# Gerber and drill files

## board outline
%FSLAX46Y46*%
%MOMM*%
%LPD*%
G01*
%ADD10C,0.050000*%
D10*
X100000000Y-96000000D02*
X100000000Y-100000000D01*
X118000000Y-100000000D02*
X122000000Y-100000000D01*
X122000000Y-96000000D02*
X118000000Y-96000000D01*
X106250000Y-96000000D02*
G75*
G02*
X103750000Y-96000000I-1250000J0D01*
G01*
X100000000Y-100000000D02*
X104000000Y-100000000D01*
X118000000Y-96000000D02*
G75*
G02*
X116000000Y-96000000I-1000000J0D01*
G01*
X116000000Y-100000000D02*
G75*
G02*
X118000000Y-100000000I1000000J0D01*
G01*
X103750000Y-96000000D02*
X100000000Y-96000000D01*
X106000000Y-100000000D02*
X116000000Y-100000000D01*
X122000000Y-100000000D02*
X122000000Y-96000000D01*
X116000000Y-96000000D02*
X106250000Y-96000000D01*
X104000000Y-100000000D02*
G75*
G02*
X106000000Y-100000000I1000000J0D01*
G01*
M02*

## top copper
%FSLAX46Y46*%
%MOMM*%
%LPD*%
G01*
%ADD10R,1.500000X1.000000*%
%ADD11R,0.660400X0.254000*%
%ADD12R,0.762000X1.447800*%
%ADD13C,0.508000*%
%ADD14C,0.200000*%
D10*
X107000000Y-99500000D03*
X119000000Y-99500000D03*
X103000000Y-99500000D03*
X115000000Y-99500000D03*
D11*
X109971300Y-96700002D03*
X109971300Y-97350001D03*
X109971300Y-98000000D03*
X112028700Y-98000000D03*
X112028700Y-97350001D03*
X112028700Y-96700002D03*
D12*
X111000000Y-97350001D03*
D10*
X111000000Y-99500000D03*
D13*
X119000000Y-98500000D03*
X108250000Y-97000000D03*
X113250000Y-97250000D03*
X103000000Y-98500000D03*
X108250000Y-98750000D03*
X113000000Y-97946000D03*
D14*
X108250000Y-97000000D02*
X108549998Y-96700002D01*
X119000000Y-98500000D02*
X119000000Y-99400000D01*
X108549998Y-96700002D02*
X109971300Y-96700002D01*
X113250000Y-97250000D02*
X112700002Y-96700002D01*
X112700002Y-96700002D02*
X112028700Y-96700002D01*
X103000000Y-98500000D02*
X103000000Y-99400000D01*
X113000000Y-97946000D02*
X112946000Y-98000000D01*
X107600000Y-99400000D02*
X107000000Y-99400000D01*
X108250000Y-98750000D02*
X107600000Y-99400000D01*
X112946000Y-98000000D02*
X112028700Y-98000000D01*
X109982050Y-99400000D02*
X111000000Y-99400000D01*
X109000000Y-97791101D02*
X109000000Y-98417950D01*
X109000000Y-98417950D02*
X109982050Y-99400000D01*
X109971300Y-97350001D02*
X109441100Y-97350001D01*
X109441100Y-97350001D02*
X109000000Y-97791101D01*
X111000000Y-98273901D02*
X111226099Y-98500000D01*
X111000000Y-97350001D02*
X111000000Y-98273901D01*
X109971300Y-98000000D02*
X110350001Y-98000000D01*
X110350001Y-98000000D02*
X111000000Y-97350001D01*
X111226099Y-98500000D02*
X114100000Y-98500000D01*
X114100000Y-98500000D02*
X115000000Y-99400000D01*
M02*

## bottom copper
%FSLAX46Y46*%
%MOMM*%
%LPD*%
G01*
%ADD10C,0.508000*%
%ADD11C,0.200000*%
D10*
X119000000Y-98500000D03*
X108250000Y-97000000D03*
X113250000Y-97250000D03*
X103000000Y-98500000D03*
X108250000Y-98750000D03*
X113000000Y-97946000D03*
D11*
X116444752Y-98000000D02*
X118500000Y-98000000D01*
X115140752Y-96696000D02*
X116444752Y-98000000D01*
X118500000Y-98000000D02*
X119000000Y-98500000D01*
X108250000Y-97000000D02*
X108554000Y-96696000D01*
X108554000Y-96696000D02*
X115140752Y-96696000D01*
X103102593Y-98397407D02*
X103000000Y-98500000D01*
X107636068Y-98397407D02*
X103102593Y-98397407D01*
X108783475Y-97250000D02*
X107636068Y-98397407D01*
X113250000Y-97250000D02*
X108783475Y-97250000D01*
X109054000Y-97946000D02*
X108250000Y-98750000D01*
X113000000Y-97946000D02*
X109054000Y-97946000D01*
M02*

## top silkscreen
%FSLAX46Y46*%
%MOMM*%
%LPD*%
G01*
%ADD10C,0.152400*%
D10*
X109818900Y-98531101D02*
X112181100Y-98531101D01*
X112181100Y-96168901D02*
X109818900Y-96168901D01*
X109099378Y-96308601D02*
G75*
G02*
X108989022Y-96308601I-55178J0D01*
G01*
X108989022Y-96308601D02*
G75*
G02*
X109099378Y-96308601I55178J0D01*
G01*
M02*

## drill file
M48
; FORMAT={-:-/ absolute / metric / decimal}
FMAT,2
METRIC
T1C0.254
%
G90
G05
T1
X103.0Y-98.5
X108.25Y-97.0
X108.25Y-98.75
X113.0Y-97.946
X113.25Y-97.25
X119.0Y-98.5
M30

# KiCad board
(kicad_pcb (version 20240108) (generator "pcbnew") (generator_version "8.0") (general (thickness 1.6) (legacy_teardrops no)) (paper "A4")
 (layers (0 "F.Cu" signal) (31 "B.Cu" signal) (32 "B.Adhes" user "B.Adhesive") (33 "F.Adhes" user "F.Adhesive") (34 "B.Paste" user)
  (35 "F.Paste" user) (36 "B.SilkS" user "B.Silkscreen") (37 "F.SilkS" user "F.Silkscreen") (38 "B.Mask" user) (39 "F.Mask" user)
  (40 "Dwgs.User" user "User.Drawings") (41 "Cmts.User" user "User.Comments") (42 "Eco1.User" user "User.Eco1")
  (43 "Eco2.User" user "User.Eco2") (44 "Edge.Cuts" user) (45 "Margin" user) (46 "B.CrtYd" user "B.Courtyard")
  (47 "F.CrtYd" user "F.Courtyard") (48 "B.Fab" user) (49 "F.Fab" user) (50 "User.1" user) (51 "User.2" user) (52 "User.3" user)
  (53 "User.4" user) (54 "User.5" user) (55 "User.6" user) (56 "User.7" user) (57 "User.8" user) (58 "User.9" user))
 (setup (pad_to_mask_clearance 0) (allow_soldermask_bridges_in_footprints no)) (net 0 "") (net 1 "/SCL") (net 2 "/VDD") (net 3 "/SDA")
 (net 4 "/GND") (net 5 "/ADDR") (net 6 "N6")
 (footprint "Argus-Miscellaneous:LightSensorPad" (layer "F.Cu") (at 107 100.5)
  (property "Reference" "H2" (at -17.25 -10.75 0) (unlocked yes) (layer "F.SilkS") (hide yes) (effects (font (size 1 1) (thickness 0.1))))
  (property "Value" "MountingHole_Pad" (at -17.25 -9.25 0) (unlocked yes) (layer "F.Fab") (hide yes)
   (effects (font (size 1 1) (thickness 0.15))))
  (pad "1" smd rect (at 0 -1) (size 1.5 1) (layers "F.Cu" "F.Paste" "F.Mask") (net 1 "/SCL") (thermal_bridge_angle 45)))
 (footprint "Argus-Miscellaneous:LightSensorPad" (layer "F.Cu") (at 119 100.5)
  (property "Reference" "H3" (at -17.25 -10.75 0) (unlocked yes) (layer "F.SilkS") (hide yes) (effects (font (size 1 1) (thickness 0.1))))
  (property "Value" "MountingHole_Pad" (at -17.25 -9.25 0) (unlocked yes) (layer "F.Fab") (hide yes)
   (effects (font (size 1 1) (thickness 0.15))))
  (pad "1" smd rect (at 0 -1) (size 1.5 1) (layers "F.Cu" "F.Paste" "F.Mask") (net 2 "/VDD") (thermal_bridge_angle 45)))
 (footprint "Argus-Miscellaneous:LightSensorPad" (layer "F.Cu") (at 103 100.5)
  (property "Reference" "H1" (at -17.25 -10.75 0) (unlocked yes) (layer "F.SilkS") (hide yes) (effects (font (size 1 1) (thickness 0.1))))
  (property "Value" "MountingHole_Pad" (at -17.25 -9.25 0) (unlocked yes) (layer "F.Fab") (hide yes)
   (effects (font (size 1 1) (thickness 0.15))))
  (pad "1" smd rect (at 0 -1) (size 1.5 1) (layers "F.Cu" "F.Paste" "F.Mask") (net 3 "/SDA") (thermal_bridge_angle 45)))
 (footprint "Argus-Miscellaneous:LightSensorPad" (layer "F.Cu") (at 115 100.5)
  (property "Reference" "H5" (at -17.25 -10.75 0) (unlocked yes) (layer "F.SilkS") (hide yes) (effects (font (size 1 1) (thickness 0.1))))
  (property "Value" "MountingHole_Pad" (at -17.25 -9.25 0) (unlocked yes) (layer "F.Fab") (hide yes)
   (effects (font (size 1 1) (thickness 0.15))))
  (pad "1" smd rect (at 0 -1) (size 1.5 1) (layers "F.Cu" "F.Paste" "F.Mask") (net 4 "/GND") (thermal_bridge_angle 45)))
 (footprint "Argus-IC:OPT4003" (layer "F.Cu") (at 111 97.350001)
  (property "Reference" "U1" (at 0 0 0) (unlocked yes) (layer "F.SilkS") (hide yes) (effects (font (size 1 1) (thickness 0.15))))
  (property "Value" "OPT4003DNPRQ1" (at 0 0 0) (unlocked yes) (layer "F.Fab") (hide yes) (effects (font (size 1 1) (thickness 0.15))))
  (fp_line (start -1.1811 1.1811) (end 1.1811 1.1811) (stroke (width 0.1524) (type solid)) (layer "F.SilkS"))
  (fp_line (start 1.1811 -1.1811) (end -1.1811 -1.1811) (stroke (width 0.1524) (type solid)) (layer "F.SilkS"))
  (fp_circle (center -1.9558 -1.0414) (end -1.9027 -1.0264) (stroke (width 0.1524) (type solid)) (fill none) (layer "F.SilkS"))
  (pad "1" smd rect (at -1.0287 -0.649999) (size 0.6604 0.254) (layers "F.Cu" "F.Paste" "F.Mask") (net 2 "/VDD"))
  (pad "2" smd rect (at -1.0287 0) (size 0.6604 0.254) (layers "F.Cu" "F.Paste" "F.Mask") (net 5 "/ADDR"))
  (pad "3" smd rect (at -1.0287 0.649999) (size 0.6604 0.254) (layers "F.Cu" "F.Paste" "F.Mask") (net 4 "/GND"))
  (pad "4" smd rect (at 1.0287 0.649999) (size 0.6604 0.254) (layers "F.Cu" "F.Paste" "F.Mask") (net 1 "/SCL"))
  (pad "5" smd rect (at 1.0287 0) (size 0.6604 0.254) (layers "F.Cu" "F.Paste" "F.Mask") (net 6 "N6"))
  (pad "6" smd rect (at 1.0287 -0.649999) (size 0.6604 0.254) (layers "F.Cu" "F.Paste" "F.Mask") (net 3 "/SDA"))
  (pad "7" smd rect (at 0 0) (size 0.762 1.4478) (layers "F.Cu" "F.Paste" "F.Mask") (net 4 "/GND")))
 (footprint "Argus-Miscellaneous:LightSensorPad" (layer "F.Cu") (at 111 100.5)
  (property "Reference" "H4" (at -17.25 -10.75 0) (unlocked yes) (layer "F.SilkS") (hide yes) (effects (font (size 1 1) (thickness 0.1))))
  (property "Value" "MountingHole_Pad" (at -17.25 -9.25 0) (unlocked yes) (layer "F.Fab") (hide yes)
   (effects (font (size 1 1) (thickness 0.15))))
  (pad "1" smd rect (at 0 -1) (size 1.5 1) (layers "F.Cu" "F.Paste" "F.Mask") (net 5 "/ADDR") (thermal_bridge_angle 45)))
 (gr_line (start 100 96) (end 100 100) (stroke (width 0.05) (type default)) (layer "Edge.Cuts"))
 (gr_line (start 118 100) (end 122 100) (stroke (width 0.05) (type default)) (layer "Edge.Cuts"))
 (gr_line (start 122 96) (end 118 96) (stroke (width 0.05) (type default)) (layer "Edge.Cuts"))
 (gr_arc (start 106.25 96) (mid 105 97.25) (end 103.75 96) (stroke (width 0.05) (type default)) (layer "Edge.Cuts"))
 (gr_line (start 100 100) (end 104 100) (stroke (width 0.05) (type default)) (layer "Edge.Cuts"))
 (gr_arc (start 118 96) (mid 117 97) (end 116 96) (stroke (width 0.05) (type default)) (layer "Edge.Cuts"))
 (gr_arc (start 116 100) (mid 117 99) (end 118 100) (stroke (width 0.05) (type default)) (layer "Edge.Cuts"))
 (gr_line (start 103.75 96) (end 100 96) (stroke (width 0.05) (type default)) (layer "Edge.Cuts"))
 (gr_line (start 106 100) (end 116 100) (stroke (width 0.05) (type default)) (layer "Edge.Cuts"))
 (gr_line (start 122 100) (end 122 96) (stroke (width 0.05) (type default)) (layer "Edge.Cuts"))
 (gr_line (start 116 96) (end 106.25 96) (stroke (width 0.05) (type default)) (layer "Edge.Cuts"))
 (gr_arc (start 104 100) (mid 105 99) (end 106 100) (stroke (width 0.05) (type default)) (layer "Edge.Cuts"))
 (segment (start 108.25 97) (end 108.549998 96.700002) (width 0.2) (layer "F.Cu") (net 2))
 (segment (start 119 98.5) (end 119 99.4) (width 0.2) (layer "F.Cu") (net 2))
 (segment (start 108.549998 96.700002) (end 109.9713 96.700002) (width 0.2) (layer "F.Cu") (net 2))
 (via (at 119 98.5) (size 0.508) (drill 0.254) (layers "F.Cu" "B.Cu") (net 2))
 (via (at 108.25 97) (size 0.508) (drill 0.254) (layers "F.Cu" "B.Cu") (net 2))
 (segment (start 116.444752 98) (end 118.5 98) (width 0.2) (layer "B.Cu") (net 2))
 (segment (start 115.140752 96.696) (end 116.444752 98) (width 0.2) (layer "B.Cu") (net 2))
 (segment (start 118.5 98) (end 119 98.5) (width 0.2) (layer "B.Cu") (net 2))
 (segment (start 108.25 97) (end 108.554 96.696) (width 0.2) (layer "B.Cu") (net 2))
 (segment (start 108.554 96.696) (end 115.140752 96.696) (width 0.2) (layer "B.Cu") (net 2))
 (segment (start 113.25 97.25) (end 112.700002 96.700002) (width 0.2) (layer "F.Cu") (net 3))
 (segment (start 112.700002 96.700002) (end 112.0287 96.700002) (width 0.2) (layer "F.Cu") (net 3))
 (segment (start 103 98.5) (end 103 99.4) (width 0.2) (layer "F.Cu") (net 3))
 (via (at 113.25 97.25) (size 0.508) (drill 0.254) (layers "F.Cu" "B.Cu") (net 3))
 (via (at 103 98.5) (size 0.508) (drill 0.254) (layers "F.Cu" "B.Cu") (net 3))
 (segment (start 103.102593 98.397407) (end 103 98.5) (width 0.2) (layer "B.Cu") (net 3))
 (segment (start 107.636068 98.397407) (end 103.102593 98.397407) (width 0.2) (layer "B.Cu") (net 3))
 (segment (start 108.783475 97.25) (end 107.636068 98.397407) (width 0.2) (layer "B.Cu") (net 3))
 (segment (start 113.25 97.25) (end 108.783475 97.25) (width 0.2) (layer "B.Cu") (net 3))
 (segment (start 113 97.946) (end 112.946 98) (width 0.2) (layer "F.Cu") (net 1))
 (segment (start 107.6 99.4) (end 107 99.4) (width 0.2) (layer "F.Cu") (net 1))
 (segment (start 108.25 98.75) (end 107.6 99.4) (width 0.2) (layer "F.Cu") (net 1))
 (segment (start 112.946 98) (end 112.0287 98) (width 0.2) (layer "F.Cu") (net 1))
 (via (at 108.25 98.75) (size 0.508) (drill 0.254) (layers "F.Cu" "B.Cu") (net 1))
 (via (at 113 97.946) (size 0.508) (drill 0.254) (layers "F.Cu" "B.Cu") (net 1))
 (segment (start 109.054 97.946) (end 108.25 98.75) (width 0.2) (layer "B.Cu") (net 1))
 (segment (start 113 97.946) (end 109.054 97.946) (width 0.2) (layer "B.Cu") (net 1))
 (segment (start 109.98205 99.4) (end 111 99.4) (width 0.2) (layer "F.Cu") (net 5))
 (segment (start 109 97.791101) (end 109 98.41795) (width 0.2) (layer "F.Cu") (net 5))
 (segment (start 109 98.41795) (end 109.98205 99.4) (width 0.2) (layer "F.Cu") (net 5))
 (segment (start 109.9713 97.350001) (end 109.4411 97.350001) (width 0.2) (layer "F.Cu") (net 5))
 (segment (start 109.4411 97.350001) (end 109 97.791101) (width 0.2) (layer "F.Cu") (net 5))
 (segment (start 111 98.273901) (end 111.226099 98.5) (width 0.2) (layer "F.Cu") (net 4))
 (segment (start 111 97.350001) (end 111 98.273901) (width 0.2) (layer "F.Cu") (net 4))
 (segment (start 109.9713 98) (end 110.350001 98) (width 0.2) (layer "F.Cu") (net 4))
 (segment (start 110.350001 98) (end 111 97.350001) (width 0.2) (layer "F.Cu") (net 4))
 (segment (start 111.226099 98.5) (end 114.1 98.5) (width 0.2) (layer "F.Cu") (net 4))
 (segment (start 114.1 98.5) (end 115 99.4) (width 0.2) (layer "F.Cu") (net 4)))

